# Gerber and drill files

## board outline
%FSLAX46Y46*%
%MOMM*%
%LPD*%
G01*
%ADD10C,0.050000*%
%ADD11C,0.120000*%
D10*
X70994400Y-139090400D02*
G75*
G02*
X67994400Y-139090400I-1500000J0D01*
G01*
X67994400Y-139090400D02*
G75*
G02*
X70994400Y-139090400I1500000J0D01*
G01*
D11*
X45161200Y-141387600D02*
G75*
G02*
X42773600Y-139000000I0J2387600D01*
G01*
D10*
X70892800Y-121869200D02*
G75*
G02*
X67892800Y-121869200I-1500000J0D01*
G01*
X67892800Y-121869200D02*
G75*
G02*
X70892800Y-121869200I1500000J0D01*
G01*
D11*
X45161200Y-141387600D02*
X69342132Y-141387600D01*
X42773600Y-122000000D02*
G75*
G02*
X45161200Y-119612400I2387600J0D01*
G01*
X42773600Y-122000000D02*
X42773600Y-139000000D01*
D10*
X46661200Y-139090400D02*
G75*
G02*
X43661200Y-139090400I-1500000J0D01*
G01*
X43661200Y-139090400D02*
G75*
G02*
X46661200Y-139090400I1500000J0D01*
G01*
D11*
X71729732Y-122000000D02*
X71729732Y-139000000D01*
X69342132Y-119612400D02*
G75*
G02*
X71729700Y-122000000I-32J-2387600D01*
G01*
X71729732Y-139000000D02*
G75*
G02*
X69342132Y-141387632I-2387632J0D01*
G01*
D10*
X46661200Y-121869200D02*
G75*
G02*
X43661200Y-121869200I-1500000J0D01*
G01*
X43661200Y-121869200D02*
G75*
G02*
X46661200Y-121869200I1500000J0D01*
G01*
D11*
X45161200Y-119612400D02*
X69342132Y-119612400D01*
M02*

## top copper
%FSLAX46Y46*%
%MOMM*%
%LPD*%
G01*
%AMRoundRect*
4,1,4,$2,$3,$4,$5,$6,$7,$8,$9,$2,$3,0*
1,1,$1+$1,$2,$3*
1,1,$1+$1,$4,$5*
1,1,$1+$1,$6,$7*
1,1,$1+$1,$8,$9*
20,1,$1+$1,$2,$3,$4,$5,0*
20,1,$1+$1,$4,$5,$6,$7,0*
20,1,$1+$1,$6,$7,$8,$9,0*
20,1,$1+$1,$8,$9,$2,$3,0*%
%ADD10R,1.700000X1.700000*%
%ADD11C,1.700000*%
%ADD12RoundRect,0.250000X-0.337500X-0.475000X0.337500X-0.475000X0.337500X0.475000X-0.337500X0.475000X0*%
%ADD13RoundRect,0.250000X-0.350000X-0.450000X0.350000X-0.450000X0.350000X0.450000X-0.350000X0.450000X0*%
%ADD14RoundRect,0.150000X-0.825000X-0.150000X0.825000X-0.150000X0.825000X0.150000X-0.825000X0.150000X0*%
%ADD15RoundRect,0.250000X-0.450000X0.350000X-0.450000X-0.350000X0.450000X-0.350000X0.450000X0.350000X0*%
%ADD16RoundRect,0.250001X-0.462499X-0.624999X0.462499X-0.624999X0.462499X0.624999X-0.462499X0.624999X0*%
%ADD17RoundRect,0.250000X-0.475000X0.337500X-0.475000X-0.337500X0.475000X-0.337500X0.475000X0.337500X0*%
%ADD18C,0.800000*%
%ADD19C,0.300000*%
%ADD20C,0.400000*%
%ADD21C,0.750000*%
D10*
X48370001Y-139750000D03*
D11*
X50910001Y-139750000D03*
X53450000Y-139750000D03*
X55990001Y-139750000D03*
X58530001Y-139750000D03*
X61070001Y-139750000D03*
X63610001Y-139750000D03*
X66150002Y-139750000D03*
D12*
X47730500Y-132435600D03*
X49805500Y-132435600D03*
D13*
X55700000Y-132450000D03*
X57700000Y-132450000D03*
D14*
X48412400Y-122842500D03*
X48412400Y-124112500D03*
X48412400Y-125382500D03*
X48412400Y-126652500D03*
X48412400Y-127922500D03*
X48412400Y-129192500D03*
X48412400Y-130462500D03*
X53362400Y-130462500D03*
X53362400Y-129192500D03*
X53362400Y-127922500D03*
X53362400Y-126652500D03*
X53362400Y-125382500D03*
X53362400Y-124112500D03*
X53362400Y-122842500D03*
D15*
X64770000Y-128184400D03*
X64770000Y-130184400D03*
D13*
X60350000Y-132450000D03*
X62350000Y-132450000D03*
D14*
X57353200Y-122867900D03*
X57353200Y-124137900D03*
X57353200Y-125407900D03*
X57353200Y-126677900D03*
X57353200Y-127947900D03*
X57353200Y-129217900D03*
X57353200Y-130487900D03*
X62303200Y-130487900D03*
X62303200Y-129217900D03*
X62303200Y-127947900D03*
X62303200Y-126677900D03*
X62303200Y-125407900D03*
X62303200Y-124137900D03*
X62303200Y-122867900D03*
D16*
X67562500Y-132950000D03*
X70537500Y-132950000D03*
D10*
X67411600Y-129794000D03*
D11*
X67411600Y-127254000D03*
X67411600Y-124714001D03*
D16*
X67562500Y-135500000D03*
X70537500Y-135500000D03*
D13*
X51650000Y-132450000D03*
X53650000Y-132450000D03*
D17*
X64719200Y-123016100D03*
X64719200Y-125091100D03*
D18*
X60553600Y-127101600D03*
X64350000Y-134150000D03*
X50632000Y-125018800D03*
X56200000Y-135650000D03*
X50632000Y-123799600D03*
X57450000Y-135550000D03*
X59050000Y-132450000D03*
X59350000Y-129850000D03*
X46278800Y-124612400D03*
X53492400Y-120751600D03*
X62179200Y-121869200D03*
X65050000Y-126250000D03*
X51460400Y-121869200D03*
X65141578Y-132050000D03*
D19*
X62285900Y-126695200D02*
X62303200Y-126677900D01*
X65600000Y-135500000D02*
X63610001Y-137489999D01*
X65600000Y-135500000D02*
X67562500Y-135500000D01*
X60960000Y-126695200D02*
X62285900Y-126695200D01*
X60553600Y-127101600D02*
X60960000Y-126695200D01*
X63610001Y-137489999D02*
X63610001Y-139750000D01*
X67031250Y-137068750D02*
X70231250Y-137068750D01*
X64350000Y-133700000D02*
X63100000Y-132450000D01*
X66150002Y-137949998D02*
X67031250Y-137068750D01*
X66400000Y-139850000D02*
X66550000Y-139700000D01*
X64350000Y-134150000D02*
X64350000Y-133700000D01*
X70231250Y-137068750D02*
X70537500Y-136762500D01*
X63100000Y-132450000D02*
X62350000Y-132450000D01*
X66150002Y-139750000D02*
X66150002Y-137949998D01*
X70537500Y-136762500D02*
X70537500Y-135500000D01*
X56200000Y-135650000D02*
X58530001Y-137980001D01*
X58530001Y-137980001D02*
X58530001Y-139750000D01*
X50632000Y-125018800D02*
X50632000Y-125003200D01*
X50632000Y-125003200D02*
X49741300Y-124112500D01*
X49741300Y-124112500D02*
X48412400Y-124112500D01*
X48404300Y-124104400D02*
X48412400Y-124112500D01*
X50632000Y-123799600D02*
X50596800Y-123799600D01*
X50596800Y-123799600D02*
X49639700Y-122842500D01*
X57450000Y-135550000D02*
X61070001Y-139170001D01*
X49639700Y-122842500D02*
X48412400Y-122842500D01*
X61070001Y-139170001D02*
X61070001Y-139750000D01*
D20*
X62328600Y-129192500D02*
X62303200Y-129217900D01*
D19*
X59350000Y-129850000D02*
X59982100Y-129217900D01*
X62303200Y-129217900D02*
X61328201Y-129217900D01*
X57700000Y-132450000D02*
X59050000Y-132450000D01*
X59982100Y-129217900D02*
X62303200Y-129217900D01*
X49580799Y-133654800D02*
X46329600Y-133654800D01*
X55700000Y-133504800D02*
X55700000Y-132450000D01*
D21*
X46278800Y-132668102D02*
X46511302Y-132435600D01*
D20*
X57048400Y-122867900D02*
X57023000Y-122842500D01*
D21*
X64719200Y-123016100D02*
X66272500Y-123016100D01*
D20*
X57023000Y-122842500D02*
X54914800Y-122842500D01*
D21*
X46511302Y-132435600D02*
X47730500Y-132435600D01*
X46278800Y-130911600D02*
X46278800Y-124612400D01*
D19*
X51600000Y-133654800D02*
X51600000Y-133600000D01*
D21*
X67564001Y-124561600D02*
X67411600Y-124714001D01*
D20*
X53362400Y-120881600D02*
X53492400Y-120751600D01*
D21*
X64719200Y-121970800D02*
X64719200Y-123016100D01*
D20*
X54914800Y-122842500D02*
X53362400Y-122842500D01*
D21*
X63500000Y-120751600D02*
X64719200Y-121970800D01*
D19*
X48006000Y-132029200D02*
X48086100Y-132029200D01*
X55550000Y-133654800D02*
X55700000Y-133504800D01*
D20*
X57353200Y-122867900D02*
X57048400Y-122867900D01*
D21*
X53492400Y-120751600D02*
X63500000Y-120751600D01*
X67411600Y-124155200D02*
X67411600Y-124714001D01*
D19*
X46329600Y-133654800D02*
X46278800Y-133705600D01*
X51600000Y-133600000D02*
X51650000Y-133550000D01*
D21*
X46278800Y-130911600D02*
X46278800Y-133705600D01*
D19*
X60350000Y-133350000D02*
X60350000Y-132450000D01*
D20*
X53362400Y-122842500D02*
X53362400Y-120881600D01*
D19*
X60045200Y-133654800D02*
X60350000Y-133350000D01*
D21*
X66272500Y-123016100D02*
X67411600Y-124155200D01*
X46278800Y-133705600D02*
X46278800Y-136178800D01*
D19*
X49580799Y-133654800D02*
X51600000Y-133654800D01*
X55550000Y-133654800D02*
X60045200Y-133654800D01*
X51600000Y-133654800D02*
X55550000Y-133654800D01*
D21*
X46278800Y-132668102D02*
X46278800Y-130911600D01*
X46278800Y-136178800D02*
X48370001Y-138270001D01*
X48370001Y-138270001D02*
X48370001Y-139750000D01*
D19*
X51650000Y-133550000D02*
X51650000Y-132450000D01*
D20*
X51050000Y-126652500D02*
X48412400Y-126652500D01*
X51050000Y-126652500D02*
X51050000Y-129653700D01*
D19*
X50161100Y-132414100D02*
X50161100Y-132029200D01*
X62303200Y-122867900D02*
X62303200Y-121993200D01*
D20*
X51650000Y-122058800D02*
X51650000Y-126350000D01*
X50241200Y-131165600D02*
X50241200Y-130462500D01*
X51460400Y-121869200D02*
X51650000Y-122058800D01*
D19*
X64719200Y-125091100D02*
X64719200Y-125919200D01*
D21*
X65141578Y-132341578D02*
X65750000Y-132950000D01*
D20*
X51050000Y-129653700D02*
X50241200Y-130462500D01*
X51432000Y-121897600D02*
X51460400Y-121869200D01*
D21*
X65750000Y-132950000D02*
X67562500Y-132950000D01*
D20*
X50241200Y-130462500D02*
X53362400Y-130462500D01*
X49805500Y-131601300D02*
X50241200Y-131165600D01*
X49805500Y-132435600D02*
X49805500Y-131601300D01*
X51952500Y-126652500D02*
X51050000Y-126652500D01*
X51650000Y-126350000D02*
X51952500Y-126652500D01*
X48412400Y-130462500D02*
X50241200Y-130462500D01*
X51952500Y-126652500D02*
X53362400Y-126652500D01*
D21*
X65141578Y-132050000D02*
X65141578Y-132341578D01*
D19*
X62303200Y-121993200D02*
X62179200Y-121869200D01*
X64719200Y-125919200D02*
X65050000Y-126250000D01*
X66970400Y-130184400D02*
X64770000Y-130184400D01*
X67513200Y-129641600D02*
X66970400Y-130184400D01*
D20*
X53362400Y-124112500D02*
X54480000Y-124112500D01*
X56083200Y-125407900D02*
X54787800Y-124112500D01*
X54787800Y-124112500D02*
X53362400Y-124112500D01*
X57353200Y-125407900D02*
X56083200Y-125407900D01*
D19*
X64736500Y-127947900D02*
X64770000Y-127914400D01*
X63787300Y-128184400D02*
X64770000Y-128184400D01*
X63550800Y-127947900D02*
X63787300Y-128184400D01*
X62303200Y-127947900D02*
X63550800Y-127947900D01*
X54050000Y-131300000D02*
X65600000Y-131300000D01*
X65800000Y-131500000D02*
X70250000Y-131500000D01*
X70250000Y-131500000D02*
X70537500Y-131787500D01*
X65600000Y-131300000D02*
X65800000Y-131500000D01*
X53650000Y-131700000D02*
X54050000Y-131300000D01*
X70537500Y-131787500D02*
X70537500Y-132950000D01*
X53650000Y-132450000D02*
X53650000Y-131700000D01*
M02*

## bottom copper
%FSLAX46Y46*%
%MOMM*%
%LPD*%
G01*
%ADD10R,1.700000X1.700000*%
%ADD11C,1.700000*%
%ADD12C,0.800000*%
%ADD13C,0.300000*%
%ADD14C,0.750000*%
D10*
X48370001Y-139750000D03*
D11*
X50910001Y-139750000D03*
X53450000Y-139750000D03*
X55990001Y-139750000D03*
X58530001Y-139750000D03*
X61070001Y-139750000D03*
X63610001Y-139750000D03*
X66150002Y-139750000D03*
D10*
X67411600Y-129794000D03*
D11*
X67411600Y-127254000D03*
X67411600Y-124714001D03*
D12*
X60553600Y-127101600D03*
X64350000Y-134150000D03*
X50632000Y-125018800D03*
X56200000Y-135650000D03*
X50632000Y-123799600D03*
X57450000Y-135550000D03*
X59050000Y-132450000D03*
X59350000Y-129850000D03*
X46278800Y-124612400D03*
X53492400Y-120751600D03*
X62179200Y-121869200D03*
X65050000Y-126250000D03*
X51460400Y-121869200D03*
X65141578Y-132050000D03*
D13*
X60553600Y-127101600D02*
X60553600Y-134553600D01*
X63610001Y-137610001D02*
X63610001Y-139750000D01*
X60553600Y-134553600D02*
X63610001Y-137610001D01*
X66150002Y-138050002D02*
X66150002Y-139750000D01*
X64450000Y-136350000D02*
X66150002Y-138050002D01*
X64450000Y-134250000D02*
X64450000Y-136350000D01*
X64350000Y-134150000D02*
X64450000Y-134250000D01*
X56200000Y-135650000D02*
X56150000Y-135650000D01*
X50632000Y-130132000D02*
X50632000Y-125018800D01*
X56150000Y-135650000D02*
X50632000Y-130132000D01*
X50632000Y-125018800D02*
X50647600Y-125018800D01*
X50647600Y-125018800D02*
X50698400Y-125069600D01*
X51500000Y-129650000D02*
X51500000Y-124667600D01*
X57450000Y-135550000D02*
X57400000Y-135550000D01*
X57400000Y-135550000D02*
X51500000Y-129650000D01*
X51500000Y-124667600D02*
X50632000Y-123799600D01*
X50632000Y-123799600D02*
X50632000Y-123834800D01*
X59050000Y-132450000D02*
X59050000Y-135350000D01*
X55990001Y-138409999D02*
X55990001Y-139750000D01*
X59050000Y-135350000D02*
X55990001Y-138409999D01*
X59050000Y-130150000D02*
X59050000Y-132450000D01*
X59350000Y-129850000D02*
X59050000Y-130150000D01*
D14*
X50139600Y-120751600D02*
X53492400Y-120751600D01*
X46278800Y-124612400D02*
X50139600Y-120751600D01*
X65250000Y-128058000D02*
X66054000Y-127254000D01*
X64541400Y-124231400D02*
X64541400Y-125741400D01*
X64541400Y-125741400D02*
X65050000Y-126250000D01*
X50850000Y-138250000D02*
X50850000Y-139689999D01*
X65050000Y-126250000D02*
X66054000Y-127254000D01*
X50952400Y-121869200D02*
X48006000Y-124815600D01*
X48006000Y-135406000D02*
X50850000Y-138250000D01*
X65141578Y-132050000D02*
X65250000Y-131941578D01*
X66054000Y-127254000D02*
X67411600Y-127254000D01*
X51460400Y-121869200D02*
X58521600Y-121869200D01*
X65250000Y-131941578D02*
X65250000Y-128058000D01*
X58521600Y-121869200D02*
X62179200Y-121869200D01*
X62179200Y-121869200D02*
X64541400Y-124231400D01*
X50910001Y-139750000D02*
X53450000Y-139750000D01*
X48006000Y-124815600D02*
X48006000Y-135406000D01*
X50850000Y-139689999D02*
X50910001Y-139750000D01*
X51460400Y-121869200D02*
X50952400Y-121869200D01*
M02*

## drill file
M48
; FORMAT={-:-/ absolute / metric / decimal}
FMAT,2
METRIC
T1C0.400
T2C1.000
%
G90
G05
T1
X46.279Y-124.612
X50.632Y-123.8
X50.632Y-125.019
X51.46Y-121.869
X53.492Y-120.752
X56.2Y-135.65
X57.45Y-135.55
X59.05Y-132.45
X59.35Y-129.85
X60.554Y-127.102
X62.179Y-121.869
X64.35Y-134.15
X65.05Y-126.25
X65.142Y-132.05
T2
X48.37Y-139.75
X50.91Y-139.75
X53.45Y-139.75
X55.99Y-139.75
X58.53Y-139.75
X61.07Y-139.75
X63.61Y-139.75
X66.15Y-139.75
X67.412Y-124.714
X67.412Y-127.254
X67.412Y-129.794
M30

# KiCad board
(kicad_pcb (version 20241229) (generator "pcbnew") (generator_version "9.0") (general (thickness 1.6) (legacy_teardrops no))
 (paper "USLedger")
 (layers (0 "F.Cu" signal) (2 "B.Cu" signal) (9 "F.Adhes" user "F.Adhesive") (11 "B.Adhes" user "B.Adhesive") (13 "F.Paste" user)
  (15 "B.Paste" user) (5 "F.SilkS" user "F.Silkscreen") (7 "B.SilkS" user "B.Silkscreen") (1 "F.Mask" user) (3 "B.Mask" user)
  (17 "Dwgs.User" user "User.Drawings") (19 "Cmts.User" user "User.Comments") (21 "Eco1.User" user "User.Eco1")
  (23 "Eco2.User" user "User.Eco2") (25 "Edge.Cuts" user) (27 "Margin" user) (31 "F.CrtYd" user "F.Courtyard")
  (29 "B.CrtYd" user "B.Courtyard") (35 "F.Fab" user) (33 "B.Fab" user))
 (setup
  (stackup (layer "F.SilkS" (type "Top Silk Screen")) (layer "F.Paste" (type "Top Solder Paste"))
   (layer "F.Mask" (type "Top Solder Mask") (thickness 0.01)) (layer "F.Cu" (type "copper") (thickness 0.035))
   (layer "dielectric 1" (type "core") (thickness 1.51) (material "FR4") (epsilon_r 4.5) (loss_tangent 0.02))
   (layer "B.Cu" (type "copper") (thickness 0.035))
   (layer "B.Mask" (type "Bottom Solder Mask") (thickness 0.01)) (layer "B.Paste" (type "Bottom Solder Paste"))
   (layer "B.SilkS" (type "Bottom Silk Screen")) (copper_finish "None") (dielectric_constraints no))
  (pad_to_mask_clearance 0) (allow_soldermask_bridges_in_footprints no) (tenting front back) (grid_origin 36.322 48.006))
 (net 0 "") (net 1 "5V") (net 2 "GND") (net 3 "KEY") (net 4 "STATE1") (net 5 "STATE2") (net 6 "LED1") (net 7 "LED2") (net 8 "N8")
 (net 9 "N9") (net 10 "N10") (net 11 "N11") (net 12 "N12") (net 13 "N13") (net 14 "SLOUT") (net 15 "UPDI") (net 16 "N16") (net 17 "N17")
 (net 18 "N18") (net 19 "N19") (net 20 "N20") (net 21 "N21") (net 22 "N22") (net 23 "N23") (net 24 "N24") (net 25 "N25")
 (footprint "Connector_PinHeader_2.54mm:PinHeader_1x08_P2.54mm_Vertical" (layer "F.Cu") (at 48.370001 139.75 90)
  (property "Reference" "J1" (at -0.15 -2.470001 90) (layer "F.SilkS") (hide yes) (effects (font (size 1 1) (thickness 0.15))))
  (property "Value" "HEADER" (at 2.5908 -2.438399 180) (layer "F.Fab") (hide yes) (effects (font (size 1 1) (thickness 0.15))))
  (pad "1" thru_hole rect (at 0 0 90) (size 1.7 1.7) (drill 1) (layers "*.Cu" "*.Mask") (remove_unused_layers no) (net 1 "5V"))
  (pad "2" thru_hole circle (at 0 2.54 90) (size 1.7 1.7) (drill 1) (layers "*.Cu" "*.Mask") (remove_unused_layers no) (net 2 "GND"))
  (pad "3" thru_hole circle (at 0 5.079999 90) (size 1.7 1.7) (drill 1) (layers "*.Cu" "*.Mask") (remove_unused_layers no) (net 2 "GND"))
  (pad "4" thru_hole circle (at 0 7.62 90) (size 1.7 1.7) (drill 1) (layers "*.Cu" "*.Mask") (remove_unused_layers no) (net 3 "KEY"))
  (pad "5" thru_hole circle (at 0 10.16 90) (size 1.7 1.7) (drill 1) (layers "*.Cu" "*.Mask") (remove_unused_layers no) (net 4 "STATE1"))
  (pad "6" thru_hole circle (at 0 12.7 90) (size 1.7 1.7) (drill 1) (layers "*.Cu" "*.Mask") (remove_unused_layers no) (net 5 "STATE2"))
  (pad "7" thru_hole circle (at 0 15.24 90) (size 1.7 1.7) (drill 1) (layers "*.Cu" "*.Mask") (remove_unused_layers no) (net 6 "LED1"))
  (pad "8" thru_hole circle (at 0 17.780001 90) (size 1.7 1.7) (drill 1) (layers "*.Cu" "*.Mask") (remove_unused_layers no) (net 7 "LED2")))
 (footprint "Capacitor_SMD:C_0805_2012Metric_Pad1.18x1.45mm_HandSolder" (layer "F.Cu") (at 48.768 132.4356)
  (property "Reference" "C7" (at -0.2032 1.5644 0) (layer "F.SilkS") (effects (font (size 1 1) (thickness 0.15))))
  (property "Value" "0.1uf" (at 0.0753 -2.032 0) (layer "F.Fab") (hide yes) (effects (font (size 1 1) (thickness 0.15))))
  (pad "1" smd roundrect (at -1.0375 0) (size 1.175 1.45) (layers "F.Cu" "F.Mask" "F.Paste") (roundrect_rratio 0.212766) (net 1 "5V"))
  (pad "2" smd roundrect (at 1.0375 0) (size 1.175 1.45) (layers "F.Cu" "F.Mask" "F.Paste") (roundrect_rratio 0.212766) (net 2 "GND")))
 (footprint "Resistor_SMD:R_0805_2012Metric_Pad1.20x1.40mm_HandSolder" (layer "F.Cu") (at 56.7 132.45)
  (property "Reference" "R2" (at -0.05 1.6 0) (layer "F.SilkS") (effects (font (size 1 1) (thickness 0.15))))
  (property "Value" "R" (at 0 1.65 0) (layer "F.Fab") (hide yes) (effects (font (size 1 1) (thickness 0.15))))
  (pad "1" smd roundrect (at -1 0) (size 1.2 1.4) (layers "F.Cu" "F.Mask" "F.Paste") (roundrect_rratio 0.208333) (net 1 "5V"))
  (pad "2" smd roundrect (at 1 0) (size 1.2 1.4) (layers "F.Cu" "F.Mask" "F.Paste") (roundrect_rratio 0.208333) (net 3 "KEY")))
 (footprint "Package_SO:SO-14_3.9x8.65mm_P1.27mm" (layer "F.Cu") (at 50.8874 126.6525)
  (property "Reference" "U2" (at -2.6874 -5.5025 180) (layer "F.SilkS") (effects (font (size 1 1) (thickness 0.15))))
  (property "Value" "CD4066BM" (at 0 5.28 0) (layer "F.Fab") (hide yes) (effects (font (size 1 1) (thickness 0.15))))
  (pad "1" smd roundrect (at -2.475 -3.81) (size 1.95 0.6) (layers "F.Cu" "F.Mask" "F.Paste") (roundrect_rratio 0.25) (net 5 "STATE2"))
  (pad "2" smd roundrect (at -2.475 -2.54) (size 1.95 0.6) (layers "F.Cu" "F.Mask" "F.Paste") (roundrect_rratio 0.25) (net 4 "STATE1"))
  (pad "3" smd roundrect (at -2.475 -1.27) (size 1.95 0.6) (layers "F.Cu" "F.Mask" "F.Paste") (roundrect_rratio 0.25) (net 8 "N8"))
  (pad "4" smd roundrect (at -2.475 0) (size 1.95 0.6) (layers "F.Cu" "F.Mask" "F.Paste") (roundrect_rratio 0.25) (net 2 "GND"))
  (pad "5" smd roundrect (at -2.475 1.27) (size 1.95 0.6) (layers "F.Cu" "F.Mask" "F.Paste") (roundrect_rratio 0.25) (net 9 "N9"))
  (pad "6" smd roundrect (at -2.475 2.54) (size 1.95 0.6) (layers "F.Cu" "F.Mask" "F.Paste") (roundrect_rratio 0.25) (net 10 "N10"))
  (pad "7" smd roundrect (at -2.475 3.81) (size 1.95 0.6) (layers "F.Cu" "F.Mask" "F.Paste") (roundrect_rratio 0.25) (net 2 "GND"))
  (pad "8" smd roundrect (at 2.475 3.81) (size 1.95 0.6) (layers "F.Cu" "F.Mask" "F.Paste") (roundrect_rratio 0.25) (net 2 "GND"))
  (pad "9" smd roundrect (at 2.475 2.54) (size 1.95 0.6) (layers "F.Cu" "F.Mask" "F.Paste") (roundrect_rratio 0.25) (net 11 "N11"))
  (pad "10" smd roundrect (at 2.475 1.27) (size 1.95 0.6) (layers "F.Cu" "F.Mask" "F.Paste") (roundrect_rratio 0.25) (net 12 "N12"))
  (pad "11" smd roundrect (at 2.475 0) (size 1.95 0.6) (layers "F.Cu" "F.Mask" "F.Paste") (roundrect_rratio 0.25) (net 2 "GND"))
  (pad "12" smd roundrect (at 2.475 -1.27) (size 1.95 0.6) (layers "F.Cu" "F.Mask" "F.Paste") (roundrect_rratio 0.25) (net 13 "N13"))
  (pad "13" smd roundrect (at 2.475 -2.54) (size 1.95 0.6) (layers "F.Cu" "F.Mask" "F.Paste") (roundrect_rratio 0.25) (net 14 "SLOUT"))
  (pad "14" smd roundrect (at 2.475 -3.81) (size 1.95 0.6) (layers "F.Cu" "F.Mask" "F.Paste") (roundrect_rratio 0.25) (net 1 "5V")))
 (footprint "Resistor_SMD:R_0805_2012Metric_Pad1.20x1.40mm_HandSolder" (layer "F.Cu") (at 64.77 129.1844 -90)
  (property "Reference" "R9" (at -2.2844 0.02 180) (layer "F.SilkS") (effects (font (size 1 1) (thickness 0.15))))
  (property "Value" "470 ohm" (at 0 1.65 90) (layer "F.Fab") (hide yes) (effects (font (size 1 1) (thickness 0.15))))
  (pad "1" smd roundrect (at -1 0 270) (size 1.2 1.4) (layers "F.Cu" "F.Mask" "F.Paste") (roundrect_rratio 0.208333) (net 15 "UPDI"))
  (pad "2" smd roundrect (at 1 0 270) (size 1.2 1.4) (layers "F.Cu" "F.Mask" "F.Paste") (roundrect_rratio 0.208333) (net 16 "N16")))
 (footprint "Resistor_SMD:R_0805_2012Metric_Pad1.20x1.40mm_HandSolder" (layer "F.Cu") (at 61.35 132.45)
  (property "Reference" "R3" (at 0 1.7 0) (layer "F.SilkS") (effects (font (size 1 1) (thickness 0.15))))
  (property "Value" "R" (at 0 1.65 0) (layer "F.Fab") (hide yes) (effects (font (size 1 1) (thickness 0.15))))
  (pad "1" smd roundrect (at -1 0) (size 1.2 1.4) (layers "F.Cu" "F.Mask" "F.Paste") (roundrect_rratio 0.208333) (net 1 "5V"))
  (pad "2" smd roundrect (at 1 0) (size 1.2 1.4) (layers "F.Cu" "F.Mask" "F.Paste") (roundrect_rratio 0.208333) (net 7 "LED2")))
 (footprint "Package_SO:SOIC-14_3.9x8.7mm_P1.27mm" (layer "F.Cu") (at 59.8282 126.6779)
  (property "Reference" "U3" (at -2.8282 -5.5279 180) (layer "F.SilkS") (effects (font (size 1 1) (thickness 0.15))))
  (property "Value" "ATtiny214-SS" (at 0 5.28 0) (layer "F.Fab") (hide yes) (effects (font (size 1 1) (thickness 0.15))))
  (pad "1" smd roundrect (at -2.475 -3.81) (size 1.95 0.6) (layers "F.Cu" "F.Mask" "F.Paste") (roundrect_rratio 0.25) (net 1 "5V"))
  (pad "2" smd roundrect (at -2.475 -2.54) (size 1.95 0.6) (layers "F.Cu" "F.Mask" "F.Paste") (roundrect_rratio 0.25) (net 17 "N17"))
  (pad "3" smd roundrect (at -2.475 -1.27) (size 1.95 0.6) (layers "F.Cu" "F.Mask" "F.Paste") (roundrect_rratio 0.25) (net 14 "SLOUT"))
  (pad "4" smd roundrect (at -2.475 0) (size 1.95 0.6) (layers "F.Cu" "F.Mask" "F.Paste") (roundrect_rratio 0.25) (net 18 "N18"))
  (pad "5" smd roundrect (at -2.475 1.27) (size 1.95 0.6) (layers "F.Cu" "F.Mask" "F.Paste") (roundrect_rratio 0.25) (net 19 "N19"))
  (pad "6" smd roundrect (at -2.475 2.54) (size 1.95 0.6) (layers "F.Cu" "F.Mask" "F.Paste") (roundrect_rratio 0.25) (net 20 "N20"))
  (pad "7" smd roundrect (at -2.475 3.81) (size 1.95 0.6) (layers "F.Cu" "F.Mask" "F.Paste") (roundrect_rratio 0.25) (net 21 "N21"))
  (pad "8" smd roundrect (at 2.475 3.81) (size 1.95 0.6) (layers "F.Cu" "F.Mask" "F.Paste") (roundrect_rratio 0.25) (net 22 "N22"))
  (pad "9" smd roundrect (at 2.475 2.54) (size 1.95 0.6) (layers "F.Cu" "F.Mask" "F.Paste") (roundrect_rratio 0.25) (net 3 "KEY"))
  (pad "10" smd roundrect (at 2.475 1.27) (size 1.95 0.6) (layers "F.Cu" "F.Mask" "F.Paste") (roundrect_rratio 0.25) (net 15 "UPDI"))
  (pad "11" smd roundrect (at 2.475 0) (size 1.95 0.6) (layers "F.Cu" "F.Mask" "F.Paste") (roundrect_rratio 0.25) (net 6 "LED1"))
  (pad "12" smd roundrect (at 2.475 -1.27) (size 1.95 0.6) (layers "F.Cu" "F.Mask" "F.Paste") (roundrect_rratio 0.25) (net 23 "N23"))
  (pad "13" smd roundrect (at 2.475 -2.54) (size 1.95 0.6) (layers "F.Cu" "F.Mask" "F.Paste") (roundrect_rratio 0.25) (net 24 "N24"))
  (pad "14" smd roundrect (at 2.475 -3.81) (size 1.95 0.6) (layers "F.Cu" "F.Mask" "F.Paste") (roundrect_rratio 0.25) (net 2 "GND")))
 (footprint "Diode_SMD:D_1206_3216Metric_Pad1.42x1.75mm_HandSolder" (layer "F.Cu") (at 69.05 132.95)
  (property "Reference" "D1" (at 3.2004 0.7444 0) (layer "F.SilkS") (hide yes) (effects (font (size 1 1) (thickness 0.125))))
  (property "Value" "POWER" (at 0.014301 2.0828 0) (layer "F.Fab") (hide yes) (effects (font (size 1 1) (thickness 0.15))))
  (pad "1" smd roundrect (at -1.4875 0) (size 1.425 1.75) (layers "F.Cu" "F.Mask" "F.Paste") (roundrect_rratio 0.175439) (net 2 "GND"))
  (pad "2" smd roundrect (at 1.4875 0) (size 1.425 1.75) (layers "F.Cu" "F.Mask" "F.Paste") (roundrect_rratio 0.175439) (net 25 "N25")))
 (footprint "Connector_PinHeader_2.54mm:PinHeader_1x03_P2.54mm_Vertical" (layer "F.Cu") (at 67.4116 129.794 180)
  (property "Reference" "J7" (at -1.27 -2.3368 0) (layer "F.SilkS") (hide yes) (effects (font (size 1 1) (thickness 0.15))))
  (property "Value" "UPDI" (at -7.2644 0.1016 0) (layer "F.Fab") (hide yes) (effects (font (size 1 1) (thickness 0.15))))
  (pad "1" thru_hole rect (at 0 0 180) (size 1.7 1.7) (drill 1) (layers "*.Cu" "*.Mask") (remove_unused_layers no) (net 16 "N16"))
  (pad "2" thru_hole circle (at 0 2.54 180) (size 1.7 1.7) (drill 1) (layers "*.Cu" "*.Mask") (remove_unused_layers no) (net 2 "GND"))
  (pad "3" thru_hole circle (at 0 5.079999 180) (size 1.7 1.7) (drill 1) (layers "*.Cu" "*.Mask") (remove_unused_layers no) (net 1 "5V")))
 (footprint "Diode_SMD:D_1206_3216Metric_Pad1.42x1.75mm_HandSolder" (layer "F.Cu") (at 69.05 135.5)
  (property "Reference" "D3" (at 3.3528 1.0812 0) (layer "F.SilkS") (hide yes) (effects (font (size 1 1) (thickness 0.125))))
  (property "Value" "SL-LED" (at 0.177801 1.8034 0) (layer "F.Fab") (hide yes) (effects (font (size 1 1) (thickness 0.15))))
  (pad "1" smd roundrect (at -1.4875 0) (size 1.425 1.75) (layers "F.Cu" "F.Mask" "F.Paste") (roundrect_rratio 0.175439) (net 6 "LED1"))
  (pad "2" smd roundrect (at 1.4875 0) (size 1.425 1.75) (layers "F.Cu" "F.Mask" "F.Paste") (roundrect_rratio 0.175439) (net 7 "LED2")))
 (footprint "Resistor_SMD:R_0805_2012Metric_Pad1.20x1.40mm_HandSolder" (layer "F.Cu") (at 52.65 132.45)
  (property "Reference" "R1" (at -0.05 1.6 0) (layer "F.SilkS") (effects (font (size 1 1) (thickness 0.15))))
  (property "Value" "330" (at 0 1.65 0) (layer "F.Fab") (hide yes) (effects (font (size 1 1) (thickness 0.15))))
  (pad "1" smd roundrect (at -1 0) (size 1.2 1.4) (layers "F.Cu" "F.Mask" "F.Paste") (roundrect_rratio 0.208333) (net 1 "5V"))
  (pad "2" smd roundrect (at 1 0) (size 1.2 1.4) (layers "F.Cu" "F.Mask" "F.Paste") (roundrect_rratio 0.208333) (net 25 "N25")))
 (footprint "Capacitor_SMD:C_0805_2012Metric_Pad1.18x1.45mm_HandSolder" (layer "F.Cu") (at 64.7192 124.0536 -90)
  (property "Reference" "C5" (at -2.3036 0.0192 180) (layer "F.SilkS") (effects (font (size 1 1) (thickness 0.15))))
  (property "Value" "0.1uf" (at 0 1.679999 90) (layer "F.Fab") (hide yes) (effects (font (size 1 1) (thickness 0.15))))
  (pad "1" smd roundrect (at -1.0375 0 270) (size 1.175 1.45) (layers "F.Cu" "F.Mask" "F.Paste") (roundrect_rratio 0.212766) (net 1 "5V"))
  (pad "2" smd roundrect (at 1.0375 0 270) (size 1.175 1.45) (layers "F.Cu" "F.Mask" "F.Paste") (roundrect_rratio 0.212766) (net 2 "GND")))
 (gr_circle (center 69.4944 139.0904) (end 70.9944 139.0904) (stroke (width 0.05) (type solid)) (fill no) (layer "Edge.Cuts"))
 (gr_arc (start 45.1612 141.3876) (mid 43.472912 140.688288) (end 42.7736 139) (stroke (width 0.12) (type solid)) (layer "Edge.Cuts"))
 (gr_circle (center 69.3928 121.8692) (end 70.8928 121.8692) (stroke (width 0.05) (type solid)) (fill no) (layer "Edge.Cuts"))
 (gr_line (start 45.1612 141.3876) (end 69.342132 141.3876) (stroke (width 0.12) (type solid)) (layer "Edge.Cuts"))
 (gr_arc (start 42.7736 122) (mid 43.472912 120.311712) (end 45.1612 119.6124) (stroke (width 0.12) (type solid)) (layer "Edge.Cuts"))
 (gr_line (start 42.7736 122) (end 42.7736 139) (stroke (width 0.12) (type solid)) (layer "Edge.Cuts"))
 (gr_circle (center 45.1612 139.0904) (end 46.6612 139.0904) (stroke (width 0.05) (type solid)) (fill no) (layer "Edge.Cuts"))
 (gr_line (start 71.729732 122) (end 71.729732 139) (stroke (width 0.12) (type solid)) (layer "Edge.Cuts"))
 (gr_arc (start 69.342132 119.6124) (mid 71.03042 120.311712) (end 71.729732 122) (stroke (width 0.12) (type solid)) (layer "Edge.Cuts"))
 (gr_arc (start 71.729732 139) (mid 71.03042 140.688288) (end 69.342132 141.3876) (stroke (width 0.12) (type solid)) (layer "Edge.Cuts"))
 (gr_circle (center 45.1612 121.8692) (end 46.6612 121.8692) (stroke (width 0.05) (type solid)) (fill no) (layer "Edge.Cuts"))
 (gr_line (start 45.1612 119.6124) (end 69.342132 119.6124) (stroke (width 0.12) (type solid)) (layer "Edge.Cuts"))
 (segment (start 62.2859 126.6952) (end 62.3032 126.6779) (width 0.3) (layer "F.Cu") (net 6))
 (segment (start 65.6 135.5) (end 63.610001 137.489999) (width 0.3) (layer "F.Cu") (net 6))
 (segment (start 65.6 135.5) (end 67.5625 135.5) (width 0.3) (layer "F.Cu") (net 6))
 (segment (start 60.96 126.6952) (end 62.2859 126.6952) (width 0.3) (layer "F.Cu") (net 6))
 (segment (start 60.5536 127.1016) (end 60.96 126.6952) (width 0.3) (layer "F.Cu") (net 6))
 (segment (start 63.610001 137.489999) (end 63.610001 139.75) (width 0.3) (layer "F.Cu") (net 6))
 (via (at 60.5536 127.1016) (size 0.8) (drill 0.4) (layers "F.Cu" "B.Cu") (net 6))
 (segment (start 60.5536 127.1016) (end 60.5536 134.5536) (width 0.3) (layer "B.Cu") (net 6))
 (segment (start 63.610001 137.610001) (end 63.610001 139.75) (width 0.3) (layer "B.Cu") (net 6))
 (segment (start 60.5536 134.5536) (end 63.610001 137.610001) (width 0.3) (layer "B.Cu") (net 6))
 (segment (start 67.03125 137.06875) (end 70.23125 137.06875) (width 0.3) (layer "F.Cu") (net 7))
 (segment (start 64.35 133.7) (end 63.1 132.45) (width 0.3) (layer "F.Cu") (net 7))
 (segment (start 66.150002 137.949998) (end 67.03125 137.06875) (width 0.3) (layer "F.Cu") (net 7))
 (segment (start 66.4 139.85) (end 66.55 139.7) (width 0.3) (layer "F.Cu") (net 7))
 (segment (start 64.35 134.15) (end 64.35 133.7) (width 0.3) (layer "F.Cu") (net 7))
 (segment (start 70.23125 137.06875) (end 70.5375 136.7625) (width 0.3) (layer "F.Cu") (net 7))
 (segment (start 63.1 132.45) (end 62.35 132.45) (width 0.3) (layer "F.Cu") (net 7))
 (segment (start 66.150002 139.75) (end 66.150002 137.949998) (width 0.3) (layer "F.Cu") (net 7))
 (segment (start 70.5375 136.7625) (end 70.5375 135.5) (width 0.3) (layer "F.Cu") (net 7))
 (via (at 64.35 134.15) (size 0.8) (drill 0.4) (layers "F.Cu" "B.Cu") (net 7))
 (segment (start 66.150002 138.050002) (end 66.150002 139.75) (width 0.3) (layer "B.Cu") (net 7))
 (segment (start 64.45 136.35) (end 66.150002 138.050002) (width 0.3) (layer "B.Cu") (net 7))
 (segment (start 64.45 134.25) (end 64.45 136.35) (width 0.3) (layer "B.Cu") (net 7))
 (segment (start 64.35 134.15) (end 64.45 134.25) (width 0.3) (layer "B.Cu") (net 7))
 (segment (start 56.2 135.65) (end 58.530001 137.980001) (width 0.3) (layer "F.Cu") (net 4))
 (segment (start 58.530001 137.980001) (end 58.530001 139.75) (width 0.3) (layer "F.Cu") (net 4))
 (segment (start 50.632 125.0188) (end 50.632 125.0032) (width 0.3) (layer "F.Cu") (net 4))
 (segment (start 50.632 125.0032) (end 49.7413 124.1125) (width 0.3) (layer "F.Cu") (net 4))
 (segment (start 49.7413 124.1125) (end 48.4124 124.1125) (width 0.3) (layer "F.Cu") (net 4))
 (segment (start 48.4043 124.1044) (end 48.4124 124.1125) (width 0.3) (layer "F.Cu") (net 4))
 (via (at 50.632 125.0188) (size 0.8) (drill 0.4) (layers "F.Cu" "B.Cu") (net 4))
 (via (at 56.2 135.65) (size 0.8) (drill 0.4) (layers "F.Cu" "B.Cu") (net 4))
 (segment (start 56.2 135.65) (end 56.15 135.65) (width 0.3) (layer "B.Cu") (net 4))
 (segment (start 50.632 130.132) (end 50.632 125.0188) (width 0.3) (layer "B.Cu") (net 4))
 (segment (start 56.15 135.65) (end 50.632 130.132) (width 0.3) (layer "B.Cu") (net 4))
 (segment (start 50.632 125.0188) (end 50.6476 125.0188) (width 0.3) (layer "B.Cu") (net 4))
 (segment (start 50.6476 125.0188) (end 50.6984 125.0696) (width 0.3) (layer "B.Cu") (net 4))
 (segment (start 50.632 123.7996) (end 50.5968 123.7996) (width 0.3) (layer "F.Cu") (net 5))
 (segment (start 50.5968 123.7996) (end 49.6397 122.8425) (width 0.3) (layer "F.Cu") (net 5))
 (segment (start 57.45 135.55) (end 61.070001 139.170001) (width 0.3) (layer "F.Cu") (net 5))
 (segment (start 49.6397 122.8425) (end 48.4124 122.8425) (width 0.3) (layer "F.Cu") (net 5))
 (segment (start 61.070001 139.170001) (end 61.070001 139.75) (width 0.3) (layer "F.Cu") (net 5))
 (via (at 50.632 123.7996) (size 0.8) (drill 0.4) (layers "F.Cu" "B.Cu") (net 5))
 (via (at 57.45 135.55) (size 0.8) (drill 0.4) (layers "F.Cu" "B.Cu") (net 5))
 (segment (start 51.5 129.65) (end 51.5 124.6676) (width 0.3) (layer "B.Cu") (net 5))
 (segment (start 57.45 135.55) (end 57.4 135.55) (width 0.3) (layer "B.Cu") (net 5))
 (segment (start 57.4 135.55) (end 51.5 129.65) (width 0.3) (layer "B.Cu") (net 5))
 (segment (start 51.5 124.6676) (end 50.632 123.7996) (width 0.3) (layer "B.Cu") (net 5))
 (segment (start 50.632 123.7996) (end 50.632 123.8348) (width 0.3) (layer "B.Cu") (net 5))
 (segment (start 62.3286 129.1925) (end 62.3032 129.2179) (width 0.4) (layer "F.Cu") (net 3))
 (segment (start 59.35 129.85) (end 59.9821 129.2179) (width 0.3) (layer "F.Cu") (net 3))
 (segment (start 62.3032 129.2179) (end 61.328201 129.2179) (width 0.3) (layer "F.Cu") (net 3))
 (segment (start 57.7 132.45) (end 59.05 132.45) (width 0.3) (layer "F.Cu") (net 3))
 (segment (start 59.9821 129.2179) (end 62.3032 129.2179) (width 0.3) (layer "F.Cu") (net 3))
 (via (at 59.05 132.45) (size 0.8) (drill 0.4) (layers "F.Cu" "B.Cu") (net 3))
 (via (at 59.35 129.85) (size 0.8) (drill 0.4) (layers "F.Cu" "B.Cu") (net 3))
 (segment (start 59.05 132.45) (end 59.05 135.35) (width 0.3) (layer "B.Cu") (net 3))
 (segment (start 55.990001 138.409999) (end 55.990001 139.75) (width 0.3) (layer "B.Cu") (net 3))
 (segment (start 59.05 135.35) (end 55.990001 138.409999) (width 0.3) (layer "B.Cu") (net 3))
 (segment (start 59.05 130.15) (end 59.05 132.45) (width 0.3) (layer "B.Cu") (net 3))
 (segment (start 59.35 129.85) (end 59.05 130.15) (width 0.3) (layer "B.Cu") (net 3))
 (segment (start 49.580799 133.6548) (end 46.3296 133.6548) (width 0.3) (layer "F.Cu") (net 1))
 (segment (start 55.7 133.5048) (end 55.7 132.45) (width 0.3) (layer "F.Cu") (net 1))
 (segment (start 46.2788 132.668102) (end 46.511302 132.4356) (width 0.75) (layer "F.Cu") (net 1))
 (segment (start 57.0484 122.8679) (end 57.023 122.8425) (width 0.4) (layer "F.Cu") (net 1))
 (segment (start 64.7192 123.0161) (end 66.2725 123.0161) (width 0.75) (layer "F.Cu") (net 1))
 (segment (start 57.023 122.8425) (end 54.9148 122.8425) (width 0.4) (layer "F.Cu") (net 1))
 (segment (start 46.511302 132.4356) (end 47.7305 132.4356) (width 0.75) (layer "F.Cu") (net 1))
 (segment (start 46.2788 130.9116) (end 46.2788 124.6124) (width 0.75) (layer "F.Cu") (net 1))
 (segment (start 51.6 133.6548) (end 51.6 133.6) (width 0.3) (layer "F.Cu") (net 1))
 (segment (start 67.564001 124.5616) (end 67.4116 124.714001) (width 0.75) (layer "F.Cu") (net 1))
 (segment (start 53.3624 120.8816) (end 53.4924 120.7516) (width 0.4) (layer "F.Cu") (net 1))
 (segment (start 64.7192 121.9708) (end 64.7192 123.0161) (width 0.75) (layer "F.Cu") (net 1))
 (segment (start 54.9148 122.8425) (end 53.3624 122.8425) (width 0.4) (layer "F.Cu") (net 1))
 (segment (start 63.5 120.7516) (end 64.7192 121.9708) (width 0.75) (layer "F.Cu") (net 1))
 (segment (start 48.006 132.0292) (end 48.0861 132.0292) (width 0.3) (layer "F.Cu") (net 1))
 (segment (start 55.55 133.6548) (end 55.7 133.5048) (width 0.3) (layer "F.Cu") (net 1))
 (segment (start 57.3532 122.8679) (end 57.0484 122.8679) (width 0.4) (layer "F.Cu") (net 1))
 (segment (start 53.4924 120.7516) (end 63.5 120.7516) (width 0.75) (layer "F.Cu") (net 1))
 (segment (start 67.4116 124.1552) (end 67.4116 124.714001) (width 0.75) (layer "F.Cu") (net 1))
 (segment (start 46.3296 133.6548) (end 46.2788 133.7056) (width 0.3) (layer "F.Cu") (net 1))
 (segment (start 51.6 133.6) (end 51.65 133.55) (width 0.3) (layer "F.Cu") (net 1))
 (segment (start 46.2788 130.9116) (end 46.2788 133.7056) (width 0.75) (layer "F.Cu") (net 1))
 (segment (start 60.35 133.35) (end 60.35 132.45) (width 0.3) (layer "F.Cu") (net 1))
 (segment (start 53.3624 122.8425) (end 53.3624 120.8816) (width 0.4) (layer "F.Cu") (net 1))
 (segment (start 60.0452 133.6548) (end 60.35 133.35) (width 0.3) (layer "F.Cu") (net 1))
 (segment (start 66.2725 123.0161) (end 67.4116 124.1552) (width 0.75) (layer "F.Cu") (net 1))
 (segment (start 46.2788 133.7056) (end 46.2788 136.1788) (width 0.75) (layer "F.Cu") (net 1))
 (segment (start 49.580799 133.6548) (end 51.6 133.6548) (width 0.3) (layer "F.Cu") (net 1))
 (segment (start 55.55 133.6548) (end 60.0452 133.6548) (width 0.3) (layer "F.Cu") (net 1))
 (segment (start 51.6 133.6548) (end 55.55 133.6548) (width 0.3) (layer "F.Cu") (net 1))
 (segment (start 46.2788 132.668102) (end 46.2788 130.9116) (width 0.75) (layer "F.Cu") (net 1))
 (segment (start 46.2788 136.1788) (end 48.370001 138.270001) (width 0.75) (layer "F.Cu") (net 1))
 (segment (start 48.370001 138.270001) (end 48.370001 139.75) (width 0.75) (layer "F.Cu") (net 1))
 (segment (start 51.65 133.55) (end 51.65 132.45) (width 0.3) (layer "F.Cu") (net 1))
 (via (at 46.2788 124.6124) (size 0.8) (drill 0.4) (layers "F.Cu" "B.Cu") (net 1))
 (via (at 53.4924 120.7516) (size 0.8) (drill 0.4) (layers "F.Cu" "B.Cu") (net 1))
 (segment (start 50.1396 120.7516) (end 53.4924 120.7516) (width 0.75) (layer "B.Cu") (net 1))
 (segment (start 46.2788 124.6124) (end 50.1396 120.7516) (width 0.75) (layer "B.Cu") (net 1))
 (segment (start 51.05 126.6525) (end 48.4124 126.6525) (width 0.4) (layer "F.Cu") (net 2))
 (segment (start 51.05 126.6525) (end 51.05 129.6537) (width 0.4) (layer "F.Cu") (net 2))
 (segment (start 50.1611 132.4141) (end 50.1611 132.0292) (width 0.3) (layer "F.Cu") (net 2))
 (segment (start 62.3032 122.8679) (end 62.3032 121.9932) (width 0.3) (layer "F.Cu") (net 2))
 (segment (start 51.65 122.0588) (end 51.65 126.35) (width 0.4) (layer "F.Cu") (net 2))
 (segment (start 50.2412 131.1656) (end 50.2412 130.4625) (width 0.4) (layer "F.Cu") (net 2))
 (segment (start 51.4604 121.8692) (end 51.65 122.0588) (width 0.4) (layer "F.Cu") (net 2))
 (segment (start 64.7192 125.0911) (end 64.7192 125.9192) (width 0.3) (layer "F.Cu") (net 2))
 (segment (start 65.141578 132.341578) (end 65.75 132.95) (width 0.75) (layer "F.Cu") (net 2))
 (segment (start 51.05 129.6537) (end 50.2412 130.4625) (width 0.4) (layer "F.Cu") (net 2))
 (segment (start 51.432 121.8976) (end 51.4604 121.8692) (width 0.4) (layer "F.Cu") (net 2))
 (segment (start 65.75 132.95) (end 67.5625 132.95) (width 0.75) (layer "F.Cu") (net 2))
 (segment (start 50.2412 130.4625) (end 53.3624 130.4625) (width 0.4) (layer "F.Cu") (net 2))
 (segment (start 49.8055 131.6013) (end 50.2412 131.1656) (width 0.4) (layer "F.Cu") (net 2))
 (segment (start 49.8055 132.4356) (end 49.8055 131.6013) (width 0.4) (layer "F.Cu") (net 2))
 (segment (start 51.9525 126.6525) (end 51.05 126.6525) (width 0.4) (layer "F.Cu") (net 2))
 (segment (start 51.65 126.35) (end 51.9525 126.6525) (width 0.4) (layer "F.Cu") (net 2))
 (segment (start 48.4124 130.4625) (end 50.2412 130.4625) (width 0.4) (layer "F.Cu") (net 2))
 (segment (start 51.9525 126.6525) (end 53.3624 126.6525) (width 0.4) (layer "F.Cu") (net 2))
 (segment (start 65.141578 132.05) (end 65.141578 132.341578) (width 0.75) (layer "F.Cu") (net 2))
 (segment (start 62.3032 121.9932) (end 62.1792 121.8692) (width 0.3) (layer "F.Cu") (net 2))
 (segment (start 64.7192 125.9192) (end 65.05 126.25) (width 0.3) (layer "F.Cu") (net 2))
 (via (at 62.1792 121.8692) (size 0.8) (drill 0.4) (layers "F.Cu" "B.Cu") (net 2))
 (via (at 65.05 126.25) (size 0.8) (drill 0.4) (layers "F.Cu" "B.Cu") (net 2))
 (via (at 51.4604 121.8692) (size 0.8) (drill 0.4) (layers "F.Cu" "B.Cu") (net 2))
 (via (at 65.141578 132.05) (size 0.8) (drill 0.4) (layers "F.Cu" "B.Cu") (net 2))
 (segment (start 65.25 128.058) (end 66.054 127.254) (width 0.75) (layer "B.Cu") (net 2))
 (segment (start 64.5414 124.2314) (end 64.5414 125.7414) (width 0.75) (layer "B.Cu") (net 2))
 (segment (start 64.5414 125.7414) (end 65.05 126.25) (width 0.75) (layer "B.Cu") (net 2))
 (segment (start 50.85 138.25) (end 50.85 139.689999) (width 0.75) (layer "B.Cu") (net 2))
 (segment (start 65.05 126.25) (end 66.054 127.254) (width 0.75) (layer "B.Cu") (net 2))
 (segment (start 50.9524 121.8692) (end 48.006 124.8156) (width 0.75) (layer "B.Cu") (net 2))
 (segment (start 48.006 135.406) (end 50.85 138.25) (width 0.75) (layer "B.Cu") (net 2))
 (segment (start 65.141578 132.05) (end 65.25 131.941578) (width 0.75) (layer "B.Cu") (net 2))
 (segment (start 66.054 127.254) (end 67.4116 127.254) (width 0.75) (layer "B.Cu") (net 2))
 (segment (start 51.4604 121.8692) (end 58.5216 121.8692) (width 0.75) (layer "B.Cu") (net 2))
 (segment (start 65.25 131.941578) (end 65.25 128.058) (width 0.75) (layer "B.Cu") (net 2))
 (segment (start 58.5216 121.8692) (end 62.1792 121.8692) (width 0.75) (layer "B.Cu") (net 2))
 (segment (start 62.1792 121.8692) (end 64.5414 124.2314) (width 0.75) (layer "B.Cu") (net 2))
 (segment (start 50.910001 139.75) (end 53.45 139.75) (width 0.75) (layer "B.Cu") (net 2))
 (segment (start 48.006 124.8156) (end 48.006 135.406) (width 0.75) (layer "B.Cu") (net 2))
 (segment (start 50.85 139.689999) (end 50.910001 139.75) (width 0.75) (layer "B.Cu") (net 2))
 (segment (start 51.4604 121.8692) (end 50.9524 121.8692) (width 0.75) (layer "B.Cu") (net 2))
 (segment (start 66.9704 130.1844) (end 64.77 130.1844) (width 0.3) (layer "F.Cu") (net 16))
 (segment (start 67.5132 129.6416) (end 66.9704 130.1844) (width 0.3) (layer "F.Cu") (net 16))
 (segment (start 53.3624 124.1125) (end 54.48 124.1125) (width 0.4) (layer "F.Cu") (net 14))
 (segment (start 56.0832 125.4079) (end 54.7878 124.1125) (width 0.4) (layer "F.Cu") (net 14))
 (segment (start 54.7878 124.1125) (end 53.3624 124.1125) (width 0.4) (layer "F.Cu") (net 14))
 (segment (start 57.3532 125.4079) (end 56.0832 125.4079) (width 0.4) (layer "F.Cu") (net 14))
 (segment (start 64.7365 127.9479) (end 64.77 127.9144) (width 0.3) (layer "F.Cu") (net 15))
 (segment (start 63.7873 128.1844) (end 64.77 128.1844) (width 0.3) (layer "F.Cu") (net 15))
 (segment (start 63.5508 127.9479) (end 63.7873 128.1844) (width 0.3) (layer "F.Cu") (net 15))
 (segment (start 62.3032 127.9479) (end 63.5508 127.9479) (width 0.3) (layer "F.Cu") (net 15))
 (segment (start 54.05 131.3) (end 65.6 131.3) (width 0.3) (layer "F.Cu") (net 25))
 (segment (start 65.8 131.5) (end 70.25 131.5) (width 0.3) (layer "F.Cu") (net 25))
 (segment (start 70.25 131.5) (end 70.5375 131.7875) (width 0.3) (layer "F.Cu") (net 25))
 (segment (start 65.6 131.3) (end 65.8 131.5) (width 0.3) (layer "F.Cu") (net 25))
 (segment (start 53.65 131.7) (end 54.05 131.3) (width 0.3) (layer "F.Cu") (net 25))
 (segment (start 70.5375 131.7875) (end 70.5375 132.95) (width 0.3) (layer "F.Cu") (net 25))
 (segment (start 53.65 132.45) (end 53.65 131.7) (width 0.3) (layer "F.Cu") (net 25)))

